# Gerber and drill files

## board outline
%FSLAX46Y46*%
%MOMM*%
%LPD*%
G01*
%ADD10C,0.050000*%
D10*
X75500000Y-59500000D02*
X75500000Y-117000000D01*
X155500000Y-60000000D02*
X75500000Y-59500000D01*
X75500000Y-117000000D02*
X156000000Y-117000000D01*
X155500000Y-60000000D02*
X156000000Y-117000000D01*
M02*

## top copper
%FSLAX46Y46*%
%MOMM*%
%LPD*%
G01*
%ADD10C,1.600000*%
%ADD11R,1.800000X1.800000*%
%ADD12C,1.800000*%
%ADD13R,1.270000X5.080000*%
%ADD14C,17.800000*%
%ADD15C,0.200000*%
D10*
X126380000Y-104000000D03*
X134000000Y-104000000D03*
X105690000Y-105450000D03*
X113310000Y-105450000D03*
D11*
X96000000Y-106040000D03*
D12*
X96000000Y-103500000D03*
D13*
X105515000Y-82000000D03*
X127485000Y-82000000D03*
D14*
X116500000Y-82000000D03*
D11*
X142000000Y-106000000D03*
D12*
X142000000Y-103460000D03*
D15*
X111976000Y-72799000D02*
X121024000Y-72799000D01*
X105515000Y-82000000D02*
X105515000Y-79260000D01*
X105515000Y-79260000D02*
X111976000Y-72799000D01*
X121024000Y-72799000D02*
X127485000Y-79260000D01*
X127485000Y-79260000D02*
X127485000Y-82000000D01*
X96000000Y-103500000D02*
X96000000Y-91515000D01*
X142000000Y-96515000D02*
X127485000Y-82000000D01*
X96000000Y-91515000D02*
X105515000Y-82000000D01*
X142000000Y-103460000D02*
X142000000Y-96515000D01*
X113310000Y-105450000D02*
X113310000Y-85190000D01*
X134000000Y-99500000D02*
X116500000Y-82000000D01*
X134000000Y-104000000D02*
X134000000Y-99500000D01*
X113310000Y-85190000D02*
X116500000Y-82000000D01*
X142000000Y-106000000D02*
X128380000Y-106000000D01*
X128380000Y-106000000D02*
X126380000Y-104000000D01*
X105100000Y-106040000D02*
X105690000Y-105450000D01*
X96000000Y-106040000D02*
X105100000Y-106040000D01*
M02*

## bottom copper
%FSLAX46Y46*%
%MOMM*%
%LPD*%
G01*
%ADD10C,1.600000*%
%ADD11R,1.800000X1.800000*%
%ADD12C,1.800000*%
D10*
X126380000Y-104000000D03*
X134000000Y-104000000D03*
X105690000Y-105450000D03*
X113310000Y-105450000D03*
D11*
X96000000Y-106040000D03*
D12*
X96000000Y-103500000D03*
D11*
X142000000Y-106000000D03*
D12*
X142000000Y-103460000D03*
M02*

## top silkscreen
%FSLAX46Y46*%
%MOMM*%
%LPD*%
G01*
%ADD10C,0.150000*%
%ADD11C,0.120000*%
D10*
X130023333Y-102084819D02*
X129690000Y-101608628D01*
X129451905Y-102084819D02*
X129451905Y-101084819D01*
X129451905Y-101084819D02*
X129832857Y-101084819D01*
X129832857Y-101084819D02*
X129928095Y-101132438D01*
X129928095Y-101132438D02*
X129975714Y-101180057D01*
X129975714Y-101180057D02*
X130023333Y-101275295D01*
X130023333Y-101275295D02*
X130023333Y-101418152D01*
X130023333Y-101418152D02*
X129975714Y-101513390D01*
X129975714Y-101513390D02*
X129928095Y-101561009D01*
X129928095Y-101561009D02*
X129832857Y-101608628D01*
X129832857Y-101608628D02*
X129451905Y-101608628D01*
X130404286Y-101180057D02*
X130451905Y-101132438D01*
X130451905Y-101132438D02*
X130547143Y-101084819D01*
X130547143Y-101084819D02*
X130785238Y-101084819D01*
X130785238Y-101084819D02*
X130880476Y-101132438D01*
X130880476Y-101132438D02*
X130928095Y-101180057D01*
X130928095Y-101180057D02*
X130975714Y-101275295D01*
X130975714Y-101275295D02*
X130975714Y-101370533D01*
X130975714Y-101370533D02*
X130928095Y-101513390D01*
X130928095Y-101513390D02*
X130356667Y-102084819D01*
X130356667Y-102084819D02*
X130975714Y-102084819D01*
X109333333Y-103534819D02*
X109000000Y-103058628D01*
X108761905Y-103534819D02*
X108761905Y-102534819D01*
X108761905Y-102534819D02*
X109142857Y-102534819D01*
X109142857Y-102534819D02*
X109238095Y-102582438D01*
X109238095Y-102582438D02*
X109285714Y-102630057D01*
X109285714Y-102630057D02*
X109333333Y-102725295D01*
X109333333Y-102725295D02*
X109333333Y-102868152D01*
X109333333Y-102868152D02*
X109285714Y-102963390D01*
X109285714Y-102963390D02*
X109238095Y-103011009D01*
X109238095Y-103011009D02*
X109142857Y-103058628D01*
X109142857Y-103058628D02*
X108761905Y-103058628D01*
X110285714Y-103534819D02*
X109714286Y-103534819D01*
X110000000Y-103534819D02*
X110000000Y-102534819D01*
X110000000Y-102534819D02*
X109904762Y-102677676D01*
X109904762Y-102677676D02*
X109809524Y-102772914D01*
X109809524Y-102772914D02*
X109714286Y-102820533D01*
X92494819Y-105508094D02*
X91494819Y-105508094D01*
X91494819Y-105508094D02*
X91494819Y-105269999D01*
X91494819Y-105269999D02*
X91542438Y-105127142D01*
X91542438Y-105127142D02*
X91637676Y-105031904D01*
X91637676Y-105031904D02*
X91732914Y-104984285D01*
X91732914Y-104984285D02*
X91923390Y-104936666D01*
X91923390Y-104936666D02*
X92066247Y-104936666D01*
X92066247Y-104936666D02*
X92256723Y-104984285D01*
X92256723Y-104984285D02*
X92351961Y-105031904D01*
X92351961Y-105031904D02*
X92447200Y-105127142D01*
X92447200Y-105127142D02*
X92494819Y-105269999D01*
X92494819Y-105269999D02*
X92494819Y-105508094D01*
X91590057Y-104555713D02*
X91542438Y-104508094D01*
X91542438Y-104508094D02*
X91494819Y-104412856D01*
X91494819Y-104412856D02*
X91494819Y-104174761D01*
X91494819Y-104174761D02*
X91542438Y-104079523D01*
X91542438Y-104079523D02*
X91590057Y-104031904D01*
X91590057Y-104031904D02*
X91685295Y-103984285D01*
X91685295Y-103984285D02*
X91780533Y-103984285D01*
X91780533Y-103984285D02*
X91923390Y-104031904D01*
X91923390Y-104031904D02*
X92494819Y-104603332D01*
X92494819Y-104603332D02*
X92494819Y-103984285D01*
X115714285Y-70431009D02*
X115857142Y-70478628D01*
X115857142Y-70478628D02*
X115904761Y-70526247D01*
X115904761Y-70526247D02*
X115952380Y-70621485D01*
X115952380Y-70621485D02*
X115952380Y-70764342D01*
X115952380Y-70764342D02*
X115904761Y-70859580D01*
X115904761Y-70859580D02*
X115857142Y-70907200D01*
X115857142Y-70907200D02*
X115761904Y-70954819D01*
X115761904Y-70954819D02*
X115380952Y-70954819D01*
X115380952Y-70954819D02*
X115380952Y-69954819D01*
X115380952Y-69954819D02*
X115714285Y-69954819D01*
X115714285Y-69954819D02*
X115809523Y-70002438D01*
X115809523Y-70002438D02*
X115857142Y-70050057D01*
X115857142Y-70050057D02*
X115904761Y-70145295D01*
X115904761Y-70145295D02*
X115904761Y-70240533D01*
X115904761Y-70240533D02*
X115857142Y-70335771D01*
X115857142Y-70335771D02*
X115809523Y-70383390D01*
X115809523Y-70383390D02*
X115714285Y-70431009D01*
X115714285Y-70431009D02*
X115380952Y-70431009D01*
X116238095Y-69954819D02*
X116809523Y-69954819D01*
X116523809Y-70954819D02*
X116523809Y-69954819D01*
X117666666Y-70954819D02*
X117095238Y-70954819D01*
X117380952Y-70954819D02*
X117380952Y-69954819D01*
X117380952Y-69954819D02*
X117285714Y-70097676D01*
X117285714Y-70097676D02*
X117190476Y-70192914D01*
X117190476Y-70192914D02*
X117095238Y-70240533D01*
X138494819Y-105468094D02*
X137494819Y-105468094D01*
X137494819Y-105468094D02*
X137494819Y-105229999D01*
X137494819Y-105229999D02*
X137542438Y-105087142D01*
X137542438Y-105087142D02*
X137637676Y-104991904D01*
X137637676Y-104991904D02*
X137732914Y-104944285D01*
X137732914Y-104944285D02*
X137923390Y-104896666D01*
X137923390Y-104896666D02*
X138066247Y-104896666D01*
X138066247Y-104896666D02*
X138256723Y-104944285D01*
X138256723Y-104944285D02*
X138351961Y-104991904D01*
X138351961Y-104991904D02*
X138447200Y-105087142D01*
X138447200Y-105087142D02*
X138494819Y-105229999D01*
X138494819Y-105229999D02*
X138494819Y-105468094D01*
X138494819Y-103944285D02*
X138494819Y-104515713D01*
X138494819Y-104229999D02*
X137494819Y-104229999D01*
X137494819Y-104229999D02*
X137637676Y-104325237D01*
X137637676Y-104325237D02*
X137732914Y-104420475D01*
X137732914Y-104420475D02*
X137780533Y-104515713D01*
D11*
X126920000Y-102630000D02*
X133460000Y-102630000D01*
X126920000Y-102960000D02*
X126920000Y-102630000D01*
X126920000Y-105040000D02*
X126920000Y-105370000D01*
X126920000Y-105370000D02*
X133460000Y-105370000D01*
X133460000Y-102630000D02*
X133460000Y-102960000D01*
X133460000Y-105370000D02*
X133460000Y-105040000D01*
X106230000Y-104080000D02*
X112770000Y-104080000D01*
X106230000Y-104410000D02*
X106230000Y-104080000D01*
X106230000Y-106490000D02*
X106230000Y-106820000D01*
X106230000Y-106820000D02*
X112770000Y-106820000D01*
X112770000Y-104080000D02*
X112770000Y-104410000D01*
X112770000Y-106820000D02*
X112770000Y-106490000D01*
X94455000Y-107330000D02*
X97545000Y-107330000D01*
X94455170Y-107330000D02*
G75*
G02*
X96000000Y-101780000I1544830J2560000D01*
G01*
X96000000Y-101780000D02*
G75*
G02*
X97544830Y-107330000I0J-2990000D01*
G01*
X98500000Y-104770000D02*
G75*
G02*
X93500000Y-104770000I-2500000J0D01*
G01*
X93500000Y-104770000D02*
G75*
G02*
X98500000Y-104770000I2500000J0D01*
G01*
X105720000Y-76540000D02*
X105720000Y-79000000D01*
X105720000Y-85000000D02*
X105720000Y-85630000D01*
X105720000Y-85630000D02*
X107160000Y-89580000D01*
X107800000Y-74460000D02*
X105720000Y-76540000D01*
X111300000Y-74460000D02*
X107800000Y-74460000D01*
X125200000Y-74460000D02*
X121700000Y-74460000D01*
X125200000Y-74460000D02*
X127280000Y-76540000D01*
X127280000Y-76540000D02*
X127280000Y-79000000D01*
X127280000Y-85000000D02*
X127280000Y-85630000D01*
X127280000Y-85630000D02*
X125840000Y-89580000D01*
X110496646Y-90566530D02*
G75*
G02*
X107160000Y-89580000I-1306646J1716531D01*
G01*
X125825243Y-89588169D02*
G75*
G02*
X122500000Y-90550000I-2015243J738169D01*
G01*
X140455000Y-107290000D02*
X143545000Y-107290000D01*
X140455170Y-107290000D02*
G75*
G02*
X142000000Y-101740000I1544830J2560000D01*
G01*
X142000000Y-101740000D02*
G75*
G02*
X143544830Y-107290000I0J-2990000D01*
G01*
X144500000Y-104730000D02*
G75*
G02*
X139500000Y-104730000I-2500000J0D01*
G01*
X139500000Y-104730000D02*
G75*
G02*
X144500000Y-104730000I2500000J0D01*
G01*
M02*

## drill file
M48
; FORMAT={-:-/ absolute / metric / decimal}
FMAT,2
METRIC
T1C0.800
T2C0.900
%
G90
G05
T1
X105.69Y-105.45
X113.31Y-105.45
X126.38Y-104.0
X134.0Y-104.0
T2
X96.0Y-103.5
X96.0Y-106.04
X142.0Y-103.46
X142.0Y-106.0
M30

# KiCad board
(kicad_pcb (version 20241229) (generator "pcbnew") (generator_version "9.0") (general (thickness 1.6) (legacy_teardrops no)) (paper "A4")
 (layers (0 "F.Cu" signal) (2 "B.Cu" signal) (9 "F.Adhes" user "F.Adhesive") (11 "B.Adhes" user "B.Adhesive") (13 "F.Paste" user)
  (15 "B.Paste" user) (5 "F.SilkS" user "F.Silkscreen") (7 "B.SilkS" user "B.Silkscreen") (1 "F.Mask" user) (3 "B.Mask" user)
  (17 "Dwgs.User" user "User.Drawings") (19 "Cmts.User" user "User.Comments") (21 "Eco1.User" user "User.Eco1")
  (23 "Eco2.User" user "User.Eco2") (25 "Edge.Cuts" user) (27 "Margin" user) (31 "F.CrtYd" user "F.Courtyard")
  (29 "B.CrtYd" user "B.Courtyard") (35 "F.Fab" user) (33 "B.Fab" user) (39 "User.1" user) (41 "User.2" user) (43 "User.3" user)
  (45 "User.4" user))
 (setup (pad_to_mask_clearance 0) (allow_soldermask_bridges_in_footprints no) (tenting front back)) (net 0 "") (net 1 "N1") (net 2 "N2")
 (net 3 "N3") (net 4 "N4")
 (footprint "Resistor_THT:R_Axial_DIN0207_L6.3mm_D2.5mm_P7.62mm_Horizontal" (layer "F.Cu") (at 126.38 104)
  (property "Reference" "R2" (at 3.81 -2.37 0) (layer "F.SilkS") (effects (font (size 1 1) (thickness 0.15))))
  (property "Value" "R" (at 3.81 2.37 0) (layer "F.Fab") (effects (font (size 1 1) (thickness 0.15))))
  (fp_line (start 0.54 -1.37) (end 7.08 -1.37) (stroke (width 0.12) (type solid)) (layer "F.SilkS"))
  (fp_line (start 0.54 -1.04) (end 0.54 -1.37) (stroke (width 0.12) (type solid)) (layer "F.SilkS"))
  (fp_line (start 0.54 1.04) (end 0.54 1.37) (stroke (width 0.12) (type solid)) (layer "F.SilkS"))
  (fp_line (start 0.54 1.37) (end 7.08 1.37) (stroke (width 0.12) (type solid)) (layer "F.SilkS"))
  (fp_line (start 7.08 -1.37) (end 7.08 -1.04) (stroke (width 0.12) (type solid)) (layer "F.SilkS"))
  (fp_line (start 7.08 1.37) (end 7.08 1.04) (stroke (width 0.12) (type solid)) (layer "F.SilkS"))
  (pad "1" thru_hole circle (at 0 0) (size 1.6 1.6) (drill 0.8) (layers "*.Cu" "*.Mask") (remove_unused_layers no) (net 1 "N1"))
  (pad "2" thru_hole circle (at 7.62 0) (size 1.6 1.6) (drill 0.8) (layers "*.Cu" "*.Mask") (remove_unused_layers no) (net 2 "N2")))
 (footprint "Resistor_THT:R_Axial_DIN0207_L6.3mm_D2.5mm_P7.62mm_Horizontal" (layer "F.Cu") (at 105.69 105.45)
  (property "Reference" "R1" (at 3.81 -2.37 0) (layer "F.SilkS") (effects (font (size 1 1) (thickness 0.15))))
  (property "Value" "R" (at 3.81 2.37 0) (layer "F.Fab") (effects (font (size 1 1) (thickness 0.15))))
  (fp_line (start 0.54 -1.37) (end 7.08 -1.37) (stroke (width 0.12) (type solid)) (layer "F.SilkS"))
  (fp_line (start 0.54 -1.04) (end 0.54 -1.37) (stroke (width 0.12) (type solid)) (layer "F.SilkS"))
  (fp_line (start 0.54 1.04) (end 0.54 1.37) (stroke (width 0.12) (type solid)) (layer "F.SilkS"))
  (fp_line (start 0.54 1.37) (end 7.08 1.37) (stroke (width 0.12) (type solid)) (layer "F.SilkS"))
  (fp_line (start 7.08 -1.37) (end 7.08 -1.04) (stroke (width 0.12) (type solid)) (layer "F.SilkS"))
  (fp_line (start 7.08 1.37) (end 7.08 1.04) (stroke (width 0.12) (type solid)) (layer "F.SilkS"))
  (pad "1" thru_hole circle (at 0 0) (size 1.6 1.6) (drill 0.8) (layers "*.Cu" "*.Mask") (remove_unused_layers no) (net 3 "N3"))
  (pad "2" thru_hole circle (at 7.62 0) (size 1.6 1.6) (drill 0.8) (layers "*.Cu" "*.Mask") (remove_unused_layers no) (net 2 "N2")))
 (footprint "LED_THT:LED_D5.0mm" (layer "F.Cu") (at 96 106.04 90)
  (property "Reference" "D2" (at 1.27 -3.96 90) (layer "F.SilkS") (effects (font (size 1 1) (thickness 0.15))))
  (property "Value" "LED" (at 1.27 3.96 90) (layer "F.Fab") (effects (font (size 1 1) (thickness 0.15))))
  (fp_line (start -1.29 -1.545) (end -1.29 1.545) (stroke (width 0.12) (type solid)) (layer "F.SilkS"))
  (fp_arc (start -1.29 -1.54483) (mid 2.071779 -2.880495) (end 4.26 0) (stroke (width 0.12) (type solid)) (layer "F.SilkS"))
  (fp_arc (start 4.26 0) (mid 2.071779 2.880495) (end -1.29 1.54483) (stroke (width 0.12) (type solid)) (layer "F.SilkS"))
  (fp_circle (center 1.27 0) (end 3.77 0) (stroke (width 0.12) (type solid)) (fill no) (layer "F.SilkS"))
  (pad "1" thru_hole rect (at 0 0 90) (size 1.8 1.8) (drill 0.9) (layers "*.Cu" "*.Mask") (remove_unused_layers no) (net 3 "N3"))
  (pad "2" thru_hole circle (at 2.54 0 90) (size 1.8 1.8) (drill 0.9) (layers "*.Cu" "*.Mask") (remove_unused_layers no) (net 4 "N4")))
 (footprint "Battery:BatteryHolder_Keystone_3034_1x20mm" (layer "F.Cu") (at 116.5 82)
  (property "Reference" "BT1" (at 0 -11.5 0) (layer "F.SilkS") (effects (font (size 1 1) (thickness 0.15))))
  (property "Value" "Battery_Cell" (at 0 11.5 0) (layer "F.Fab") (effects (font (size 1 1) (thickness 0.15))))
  (fp_line (start -10.78 -5.46) (end -10.78 -3) (stroke (width 0.12) (type solid)) (layer "F.SilkS"))
  (fp_line (start -10.78 3) (end -10.78 3.63) (stroke (width 0.12) (type solid)) (layer "F.SilkS"))
  (fp_line (start -10.78 3.63) (end -9.34 7.58) (stroke (width 0.12) (type solid)) (layer "F.SilkS"))
  (fp_line (start -8.7 -7.54) (end -10.78 -5.46) (stroke (width 0.12) (type solid)) (layer "F.SilkS"))
  (fp_line (start -5.2 -7.54) (end -8.7 -7.54) (stroke (width 0.12) (type solid)) (layer "F.SilkS"))
  (fp_line (start 8.7 -7.54) (end 5.2 -7.54) (stroke (width 0.12) (type solid)) (layer "F.SilkS"))
  (fp_line (start 8.7 -7.54) (end 10.78 -5.46) (stroke (width 0.12) (type solid)) (layer "F.SilkS"))
  (fp_line (start 10.78 -5.46) (end 10.78 -3) (stroke (width 0.12) (type solid)) (layer "F.SilkS"))
  (fp_line (start 10.78 3) (end 10.78 3.63) (stroke (width 0.12) (type solid)) (layer "F.SilkS"))
  (fp_line (start 10.78 3.63) (end 9.34 7.58) (stroke (width 0.12) (type solid)) (layer "F.SilkS"))
  (fp_arc (start -6.003354 8.56653) (mid -7.921654 8.918738) (end -9.34 7.58) (stroke (width 0.12) (type solid)) (layer "F.SilkS"))
  (fp_arc (start 9.325243 7.588169) (mid 7.90634 8.911668) (end 6 8.55) (stroke (width 0.12) (type solid)) (layer "F.SilkS"))
  (pad "1" smd rect (at -10.985 0) (size 1.27 5.08) (layers "F.Cu" "F.Mask" "F.Paste") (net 4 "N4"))
  (pad "1" smd rect (at 10.985 0) (size 1.27 5.08) (layers "F.Cu" "F.Mask" "F.Paste") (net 4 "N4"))
  (pad "2" smd circle (at 0 0) (size 17.8 17.8) (layers "F.Cu" "F.Mask") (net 2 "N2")))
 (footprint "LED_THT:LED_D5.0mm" (layer "F.Cu") (at 142 106 90)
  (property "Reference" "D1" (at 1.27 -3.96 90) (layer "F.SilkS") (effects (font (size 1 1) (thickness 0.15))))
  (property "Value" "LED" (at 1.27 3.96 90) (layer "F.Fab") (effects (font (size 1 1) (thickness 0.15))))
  (fp_line (start -1.29 -1.545) (end -1.29 1.545) (stroke (width 0.12) (type solid)) (layer "F.SilkS"))
  (fp_arc (start -1.29 -1.54483) (mid 2.071779 -2.880495) (end 4.26 0) (stroke (width 0.12) (type solid)) (layer "F.SilkS"))
  (fp_arc (start 4.26 0) (mid 2.071779 2.880495) (end -1.29 1.54483) (stroke (width 0.12) (type solid)) (layer "F.SilkS"))
  (fp_circle (center 1.27 0) (end 3.77 0) (stroke (width 0.12) (type solid)) (fill no) (layer "F.SilkS"))
  (pad "1" thru_hole rect (at 0 0 90) (size 1.8 1.8) (drill 0.9) (layers "*.Cu" "*.Mask") (remove_unused_layers no) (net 1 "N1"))
  (pad "2" thru_hole circle (at 2.54 0 90) (size 1.8 1.8) (drill 0.9) (layers "*.Cu" "*.Mask") (remove_unused_layers no) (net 4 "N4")))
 (gr_line (start 75.5 59.5) (end 75.5 117) (stroke (width 0.05) (type default)) (layer "Edge.Cuts"))
 (gr_line (start 155.5 60) (end 75.5 59.5) (stroke (width 0.05) (type default)) (layer "Edge.Cuts"))
 (gr_line (start 75.5 117) (end 156 117) (stroke (width 0.05) (type default)) (layer "Edge.Cuts"))
 (gr_line (start 155.5 60) (end 156 117) (stroke (width 0.05) (type default)) (layer "Edge.Cuts"))
 (segment (start 111.976 72.799) (end 121.024 72.799) (width 0.2) (layer "F.Cu") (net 4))
 (segment (start 105.515 82) (end 105.515 79.26) (width 0.2) (layer "F.Cu") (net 4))
 (segment (start 105.515 79.26) (end 111.976 72.799) (width 0.2) (layer "F.Cu") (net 4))
 (segment (start 121.024 72.799) (end 127.485 79.26) (width 0.2) (layer "F.Cu") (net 4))
 (segment (start 127.485 79.26) (end 127.485 82) (width 0.2) (layer "F.Cu") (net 4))
 (segment (start 96 103.5) (end 96 91.515) (width 0.2) (layer "F.Cu") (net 4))
 (segment (start 142 96.515) (end 127.485 82) (width 0.2) (layer "F.Cu") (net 4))
 (segment (start 96 91.515) (end 105.515 82) (width 0.2) (layer "F.Cu") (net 4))
 (segment (start 142 103.46) (end 142 96.515) (width 0.2) (layer "F.Cu") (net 4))
 (segment (start 113.31 105.45) (end 113.31 85.19) (width 0.2) (layer "F.Cu") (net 2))
 (segment (start 134 99.5) (end 116.5 82) (width 0.2) (layer "F.Cu") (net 2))
 (segment (start 134 104) (end 134 99.5) (width 0.2) (layer "F.Cu") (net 2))
 (segment (start 113.31 85.19) (end 116.5 82) (width 0.2) (layer "F.Cu") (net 2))
 (segment (start 142 106) (end 128.38 106) (width 0.2) (layer "F.Cu") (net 1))
 (segment (start 128.38 106) (end 126.38 104) (width 0.2) (layer "F.Cu") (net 1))
 (segment (start 105.1 106.04) (end 105.69 105.45) (width 0.2) (layer "F.Cu") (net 3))
 (segment (start 96 106.04) (end 105.1 106.04) (width 0.2) (layer "F.Cu") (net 3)))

